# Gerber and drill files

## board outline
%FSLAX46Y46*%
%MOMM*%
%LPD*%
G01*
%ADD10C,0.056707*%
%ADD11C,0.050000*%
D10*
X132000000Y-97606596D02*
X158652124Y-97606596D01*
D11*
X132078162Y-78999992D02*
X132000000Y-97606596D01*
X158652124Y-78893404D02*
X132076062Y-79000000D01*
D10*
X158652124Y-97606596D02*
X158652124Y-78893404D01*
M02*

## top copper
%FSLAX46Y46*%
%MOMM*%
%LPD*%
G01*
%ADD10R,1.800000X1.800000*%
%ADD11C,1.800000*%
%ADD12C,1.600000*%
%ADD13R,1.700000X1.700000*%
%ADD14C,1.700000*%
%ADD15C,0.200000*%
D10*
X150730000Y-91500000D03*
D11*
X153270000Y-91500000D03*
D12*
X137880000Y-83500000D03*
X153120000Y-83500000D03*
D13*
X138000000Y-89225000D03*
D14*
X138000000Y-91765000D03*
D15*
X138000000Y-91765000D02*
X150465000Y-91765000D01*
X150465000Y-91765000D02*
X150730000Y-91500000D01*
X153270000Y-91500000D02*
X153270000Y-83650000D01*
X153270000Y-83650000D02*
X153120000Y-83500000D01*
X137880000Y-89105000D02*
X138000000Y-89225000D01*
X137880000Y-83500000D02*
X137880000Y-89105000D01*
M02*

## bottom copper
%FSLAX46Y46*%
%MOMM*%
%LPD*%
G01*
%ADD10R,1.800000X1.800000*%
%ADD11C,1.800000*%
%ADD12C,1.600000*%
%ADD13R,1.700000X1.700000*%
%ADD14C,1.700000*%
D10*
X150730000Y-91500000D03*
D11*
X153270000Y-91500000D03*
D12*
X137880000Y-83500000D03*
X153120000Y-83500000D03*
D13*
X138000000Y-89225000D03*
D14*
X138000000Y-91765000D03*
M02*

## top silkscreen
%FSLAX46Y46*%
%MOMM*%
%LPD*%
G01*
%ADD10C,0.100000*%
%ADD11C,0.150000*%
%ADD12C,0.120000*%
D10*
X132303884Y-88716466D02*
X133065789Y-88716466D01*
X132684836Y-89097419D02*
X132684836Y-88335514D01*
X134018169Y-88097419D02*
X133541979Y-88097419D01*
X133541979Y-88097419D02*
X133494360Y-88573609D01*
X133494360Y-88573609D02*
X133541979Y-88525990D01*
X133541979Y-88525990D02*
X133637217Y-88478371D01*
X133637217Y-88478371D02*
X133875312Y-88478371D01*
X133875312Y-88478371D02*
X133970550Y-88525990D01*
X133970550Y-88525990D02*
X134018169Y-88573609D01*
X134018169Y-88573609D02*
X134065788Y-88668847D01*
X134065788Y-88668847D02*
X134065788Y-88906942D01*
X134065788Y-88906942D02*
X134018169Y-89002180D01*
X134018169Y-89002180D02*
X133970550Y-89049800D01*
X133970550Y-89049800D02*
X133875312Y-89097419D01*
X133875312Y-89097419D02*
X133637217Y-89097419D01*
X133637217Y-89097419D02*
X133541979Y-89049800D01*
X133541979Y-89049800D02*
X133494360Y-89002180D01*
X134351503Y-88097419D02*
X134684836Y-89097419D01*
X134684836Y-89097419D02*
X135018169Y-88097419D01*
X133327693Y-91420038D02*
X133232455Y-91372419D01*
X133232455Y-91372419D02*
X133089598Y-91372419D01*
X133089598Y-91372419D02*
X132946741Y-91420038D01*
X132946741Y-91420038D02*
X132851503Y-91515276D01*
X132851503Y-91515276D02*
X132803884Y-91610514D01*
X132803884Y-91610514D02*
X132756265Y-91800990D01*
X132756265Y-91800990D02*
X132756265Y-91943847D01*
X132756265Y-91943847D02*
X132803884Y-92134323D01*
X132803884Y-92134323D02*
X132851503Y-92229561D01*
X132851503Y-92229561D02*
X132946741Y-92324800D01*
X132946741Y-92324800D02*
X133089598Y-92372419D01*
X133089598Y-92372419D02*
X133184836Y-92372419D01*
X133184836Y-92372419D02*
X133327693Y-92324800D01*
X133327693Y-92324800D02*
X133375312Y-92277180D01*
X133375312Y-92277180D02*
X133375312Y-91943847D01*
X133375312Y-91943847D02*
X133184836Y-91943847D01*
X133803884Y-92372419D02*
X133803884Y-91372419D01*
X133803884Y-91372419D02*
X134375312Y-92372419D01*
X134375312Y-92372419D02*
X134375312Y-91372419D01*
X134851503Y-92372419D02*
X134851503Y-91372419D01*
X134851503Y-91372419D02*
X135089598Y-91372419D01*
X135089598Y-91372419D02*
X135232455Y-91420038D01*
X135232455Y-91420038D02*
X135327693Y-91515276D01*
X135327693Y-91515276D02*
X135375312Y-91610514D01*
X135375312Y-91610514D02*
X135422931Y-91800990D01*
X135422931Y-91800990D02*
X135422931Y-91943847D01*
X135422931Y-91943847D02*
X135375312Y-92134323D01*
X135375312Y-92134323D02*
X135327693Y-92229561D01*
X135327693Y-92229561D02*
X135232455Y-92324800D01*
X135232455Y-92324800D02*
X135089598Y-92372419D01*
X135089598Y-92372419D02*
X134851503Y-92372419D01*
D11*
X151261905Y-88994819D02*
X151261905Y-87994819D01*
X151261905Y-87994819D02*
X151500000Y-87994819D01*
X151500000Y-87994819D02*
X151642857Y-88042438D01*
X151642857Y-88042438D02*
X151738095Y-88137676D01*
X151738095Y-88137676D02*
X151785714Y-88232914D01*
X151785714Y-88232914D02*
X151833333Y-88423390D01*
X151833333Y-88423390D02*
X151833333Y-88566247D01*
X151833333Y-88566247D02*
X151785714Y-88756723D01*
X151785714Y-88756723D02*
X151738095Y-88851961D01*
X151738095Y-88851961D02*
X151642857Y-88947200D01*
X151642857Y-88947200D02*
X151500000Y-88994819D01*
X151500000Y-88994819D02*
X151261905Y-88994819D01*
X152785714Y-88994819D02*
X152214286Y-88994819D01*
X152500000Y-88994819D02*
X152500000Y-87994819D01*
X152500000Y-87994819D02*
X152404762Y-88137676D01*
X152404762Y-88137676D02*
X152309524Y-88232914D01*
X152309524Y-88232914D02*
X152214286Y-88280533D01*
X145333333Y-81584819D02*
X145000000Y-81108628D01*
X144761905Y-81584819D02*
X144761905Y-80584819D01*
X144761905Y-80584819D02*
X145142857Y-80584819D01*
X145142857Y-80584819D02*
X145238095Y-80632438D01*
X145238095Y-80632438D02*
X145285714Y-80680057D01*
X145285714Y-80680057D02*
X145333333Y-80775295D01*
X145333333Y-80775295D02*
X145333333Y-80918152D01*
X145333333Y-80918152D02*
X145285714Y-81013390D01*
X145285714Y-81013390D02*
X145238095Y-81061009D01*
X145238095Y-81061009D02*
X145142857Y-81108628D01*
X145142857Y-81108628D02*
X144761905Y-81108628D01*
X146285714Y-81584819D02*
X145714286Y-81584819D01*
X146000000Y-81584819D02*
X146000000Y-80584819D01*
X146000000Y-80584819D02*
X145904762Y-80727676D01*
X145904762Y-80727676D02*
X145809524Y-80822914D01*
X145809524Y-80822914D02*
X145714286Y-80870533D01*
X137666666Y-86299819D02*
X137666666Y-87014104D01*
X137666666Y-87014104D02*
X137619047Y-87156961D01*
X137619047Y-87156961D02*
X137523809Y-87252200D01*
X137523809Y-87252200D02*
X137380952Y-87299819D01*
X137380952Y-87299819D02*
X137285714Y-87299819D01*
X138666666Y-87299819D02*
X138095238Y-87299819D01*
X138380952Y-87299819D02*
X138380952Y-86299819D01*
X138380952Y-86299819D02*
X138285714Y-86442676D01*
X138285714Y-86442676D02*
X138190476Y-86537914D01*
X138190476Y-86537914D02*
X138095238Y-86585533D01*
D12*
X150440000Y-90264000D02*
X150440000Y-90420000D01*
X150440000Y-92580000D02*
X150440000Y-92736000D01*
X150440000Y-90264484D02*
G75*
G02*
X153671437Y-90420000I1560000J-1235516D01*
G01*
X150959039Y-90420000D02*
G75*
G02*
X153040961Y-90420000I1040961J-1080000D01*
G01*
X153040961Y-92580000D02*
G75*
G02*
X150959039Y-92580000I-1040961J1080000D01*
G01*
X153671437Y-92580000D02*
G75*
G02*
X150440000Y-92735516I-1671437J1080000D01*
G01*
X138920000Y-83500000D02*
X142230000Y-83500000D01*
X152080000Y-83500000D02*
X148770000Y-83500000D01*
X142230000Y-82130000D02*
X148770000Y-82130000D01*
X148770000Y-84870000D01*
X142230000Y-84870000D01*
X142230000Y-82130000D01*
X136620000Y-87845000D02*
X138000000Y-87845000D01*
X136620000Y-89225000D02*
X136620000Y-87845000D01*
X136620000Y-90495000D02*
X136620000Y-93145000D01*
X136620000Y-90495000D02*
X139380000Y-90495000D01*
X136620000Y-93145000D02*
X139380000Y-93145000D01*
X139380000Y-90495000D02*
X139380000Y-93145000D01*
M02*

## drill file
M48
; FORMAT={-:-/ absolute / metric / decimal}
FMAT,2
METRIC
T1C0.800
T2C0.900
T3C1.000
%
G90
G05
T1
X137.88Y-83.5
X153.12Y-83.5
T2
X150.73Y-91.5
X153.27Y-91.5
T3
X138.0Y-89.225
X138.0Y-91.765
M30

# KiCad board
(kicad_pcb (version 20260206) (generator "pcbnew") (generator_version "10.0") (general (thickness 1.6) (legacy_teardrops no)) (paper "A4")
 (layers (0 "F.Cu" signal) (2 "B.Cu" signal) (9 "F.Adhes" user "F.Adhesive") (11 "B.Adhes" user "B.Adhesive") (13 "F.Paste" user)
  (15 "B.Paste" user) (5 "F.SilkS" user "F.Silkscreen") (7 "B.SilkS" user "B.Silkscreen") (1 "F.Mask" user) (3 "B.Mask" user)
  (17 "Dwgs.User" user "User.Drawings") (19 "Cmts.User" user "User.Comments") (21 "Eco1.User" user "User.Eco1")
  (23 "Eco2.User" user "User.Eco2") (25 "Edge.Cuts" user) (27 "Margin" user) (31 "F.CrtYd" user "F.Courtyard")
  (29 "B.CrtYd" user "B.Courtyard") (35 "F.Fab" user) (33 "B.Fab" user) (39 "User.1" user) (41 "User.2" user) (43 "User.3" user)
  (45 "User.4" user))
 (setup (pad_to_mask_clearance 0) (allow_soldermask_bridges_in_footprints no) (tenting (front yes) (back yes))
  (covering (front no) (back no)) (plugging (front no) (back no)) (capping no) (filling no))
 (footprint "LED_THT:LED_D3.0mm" (layer "F.Cu") (at 150.73 91.5)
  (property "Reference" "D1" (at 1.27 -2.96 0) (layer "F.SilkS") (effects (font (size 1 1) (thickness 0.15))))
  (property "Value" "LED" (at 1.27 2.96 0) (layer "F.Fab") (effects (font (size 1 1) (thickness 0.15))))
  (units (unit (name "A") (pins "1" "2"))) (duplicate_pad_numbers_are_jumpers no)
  (fp_line (start -0.29 -1.236) (end -0.29 -1.08) (stroke (width 0.12) (type solid)) (layer "F.SilkS"))
  (fp_line (start -0.29 1.08) (end -0.29 1.236) (stroke (width 0.12) (type solid)) (layer "F.SilkS"))
  (fp_arc (start -0.29 -1.235516) (mid 1.36566 -1.987699) (end 2.941437 -1.08) (stroke (width 0.12) (type solid)) (layer "F.SilkS"))
  (fp_arc (start 0.229039 -1.08) (mid 1.27 -1.5) (end 2.310961 -1.08) (stroke (width 0.12) (type solid)) (layer "F.SilkS"))
  (fp_arc (start 2.310961 1.08) (mid 1.27 1.5) (end 0.229039 1.08) (stroke (width 0.12) (type solid)) (layer "F.SilkS"))
  (fp_arc (start 2.941437 1.08) (mid 1.36566 1.987699) (end -0.29 1.235516) (stroke (width 0.12) (type solid)) (layer "F.SilkS"))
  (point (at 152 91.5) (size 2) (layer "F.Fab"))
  (pad "1" thru_hole rect (at 0 0) (size 1.8 1.8) (drill 0.9) (layers "*.Cu" "*.Mask") (remove_unused_layers no) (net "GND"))
  (pad "2" thru_hole circle (at 2.54 0) (size 1.8 1.8) (drill 0.9) (layers "*.Cu" "*.Mask") (remove_unused_layers no) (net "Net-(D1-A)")))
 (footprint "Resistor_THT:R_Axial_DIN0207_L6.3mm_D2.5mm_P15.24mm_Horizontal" (layer "F.Cu") (at 137.88 83.5)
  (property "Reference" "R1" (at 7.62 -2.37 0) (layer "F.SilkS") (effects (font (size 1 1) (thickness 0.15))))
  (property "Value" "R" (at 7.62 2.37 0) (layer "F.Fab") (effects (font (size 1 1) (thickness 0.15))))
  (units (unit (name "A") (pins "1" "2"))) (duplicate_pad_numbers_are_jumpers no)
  (fp_line (start 1.04 0) (end 4.35 0) (stroke (width 0.12) (type solid)) (layer "F.SilkS"))
  (fp_line (start 14.2 0) (end 10.89 0) (stroke (width 0.12) (type solid)) (layer "F.SilkS"))
  (fp_rect (start 4.35 -1.37) (end 10.89 1.37) (stroke (width 0.12) (type solid)) (fill no) (layer "F.SilkS"))
  (pad "1" thru_hole circle (at 0 0) (size 1.6 1.6) (drill 0.8) (layers "*.Cu" "*.Mask") (remove_unused_layers no) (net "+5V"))
  (pad "2" thru_hole circle (at 15.24 0) (size 1.6 1.6) (drill 0.8) (layers "*.Cu" "*.Mask") (remove_unused_layers no) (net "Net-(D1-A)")))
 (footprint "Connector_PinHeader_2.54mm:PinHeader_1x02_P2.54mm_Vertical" (layer "F.Cu") (at 138 89.225)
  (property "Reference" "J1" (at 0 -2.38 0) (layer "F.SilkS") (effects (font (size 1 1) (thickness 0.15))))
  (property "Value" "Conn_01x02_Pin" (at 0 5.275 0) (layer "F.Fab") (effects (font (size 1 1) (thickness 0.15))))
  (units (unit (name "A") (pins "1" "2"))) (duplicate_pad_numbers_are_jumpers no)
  (fp_line (start -1.38 -1.38) (end 0 -1.38) (stroke (width 0.12) (type solid)) (layer "F.SilkS"))
  (fp_line (start -1.38 0) (end -1.38 -1.38) (stroke (width 0.12) (type solid)) (layer "F.SilkS"))
  (fp_line (start -1.38 1.27) (end -1.38 3.92) (stroke (width 0.12) (type solid)) (layer "F.SilkS"))
  (fp_line (start -1.38 1.27) (end 1.38 1.27) (stroke (width 0.12) (type solid)) (layer "F.SilkS"))
  (fp_line (start -1.38 3.92) (end 1.38 3.92) (stroke (width 0.12) (type solid)) (layer "F.SilkS"))
  (fp_line (start 1.38 1.27) (end 1.38 3.92) (stroke (width 0.12) (type solid)) (layer "F.SilkS"))
  (pad "1" thru_hole rect (at 0 0) (size 1.7 1.7) (drill 1) (layers "*.Cu" "*.Mask") (remove_unused_layers no) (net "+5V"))
  (pad "2" thru_hole circle (at 0 2.54) (size 1.7 1.7) (drill 1) (layers "*.Cu" "*.Mask") (remove_unused_layers no) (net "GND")))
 (gr_line (start 132 97.606596) (end 158.652124 97.606596) (stroke (width 0.056707) (type default)) (layer "Edge.Cuts"))
 (gr_line (start 132.078162 78.999992) (end 132 97.606596) (stroke (width 0.05) (type default)) (layer "Edge.Cuts"))
 (gr_line (start 158.652124 78.893404) (end 132.076062 79) (stroke (width 0.05) (type default)) (layer "Edge.Cuts"))
 (gr_line (start 158.652124 97.606596) (end 158.652124 78.893404) (stroke (width 0.056707) (type default)) (layer "Edge.Cuts"))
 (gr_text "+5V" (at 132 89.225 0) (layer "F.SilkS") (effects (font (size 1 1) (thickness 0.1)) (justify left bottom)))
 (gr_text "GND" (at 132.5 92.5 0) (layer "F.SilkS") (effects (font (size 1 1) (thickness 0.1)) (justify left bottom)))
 (segment (start 138 91.765) (end 150.465 91.765) (width 0.2) (layer "F.Cu") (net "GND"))
 (segment (start 150.465 91.765) (end 150.73 91.5) (width 0.2) (layer "F.Cu") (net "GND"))
 (segment (start 153.27 91.5) (end 153.27 83.65) (width 0.2) (layer "F.Cu") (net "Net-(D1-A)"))
 (segment (start 153.27 83.65) (end 153.12 83.5) (width 0.2) (layer "F.Cu") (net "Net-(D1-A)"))
 (segment (start 137.88 89.105) (end 138 89.225) (width 0.2) (layer "F.Cu") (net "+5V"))
 (segment (start 137.88 83.5) (end 137.88 89.105) (width 0.2) (layer "F.Cu") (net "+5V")))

